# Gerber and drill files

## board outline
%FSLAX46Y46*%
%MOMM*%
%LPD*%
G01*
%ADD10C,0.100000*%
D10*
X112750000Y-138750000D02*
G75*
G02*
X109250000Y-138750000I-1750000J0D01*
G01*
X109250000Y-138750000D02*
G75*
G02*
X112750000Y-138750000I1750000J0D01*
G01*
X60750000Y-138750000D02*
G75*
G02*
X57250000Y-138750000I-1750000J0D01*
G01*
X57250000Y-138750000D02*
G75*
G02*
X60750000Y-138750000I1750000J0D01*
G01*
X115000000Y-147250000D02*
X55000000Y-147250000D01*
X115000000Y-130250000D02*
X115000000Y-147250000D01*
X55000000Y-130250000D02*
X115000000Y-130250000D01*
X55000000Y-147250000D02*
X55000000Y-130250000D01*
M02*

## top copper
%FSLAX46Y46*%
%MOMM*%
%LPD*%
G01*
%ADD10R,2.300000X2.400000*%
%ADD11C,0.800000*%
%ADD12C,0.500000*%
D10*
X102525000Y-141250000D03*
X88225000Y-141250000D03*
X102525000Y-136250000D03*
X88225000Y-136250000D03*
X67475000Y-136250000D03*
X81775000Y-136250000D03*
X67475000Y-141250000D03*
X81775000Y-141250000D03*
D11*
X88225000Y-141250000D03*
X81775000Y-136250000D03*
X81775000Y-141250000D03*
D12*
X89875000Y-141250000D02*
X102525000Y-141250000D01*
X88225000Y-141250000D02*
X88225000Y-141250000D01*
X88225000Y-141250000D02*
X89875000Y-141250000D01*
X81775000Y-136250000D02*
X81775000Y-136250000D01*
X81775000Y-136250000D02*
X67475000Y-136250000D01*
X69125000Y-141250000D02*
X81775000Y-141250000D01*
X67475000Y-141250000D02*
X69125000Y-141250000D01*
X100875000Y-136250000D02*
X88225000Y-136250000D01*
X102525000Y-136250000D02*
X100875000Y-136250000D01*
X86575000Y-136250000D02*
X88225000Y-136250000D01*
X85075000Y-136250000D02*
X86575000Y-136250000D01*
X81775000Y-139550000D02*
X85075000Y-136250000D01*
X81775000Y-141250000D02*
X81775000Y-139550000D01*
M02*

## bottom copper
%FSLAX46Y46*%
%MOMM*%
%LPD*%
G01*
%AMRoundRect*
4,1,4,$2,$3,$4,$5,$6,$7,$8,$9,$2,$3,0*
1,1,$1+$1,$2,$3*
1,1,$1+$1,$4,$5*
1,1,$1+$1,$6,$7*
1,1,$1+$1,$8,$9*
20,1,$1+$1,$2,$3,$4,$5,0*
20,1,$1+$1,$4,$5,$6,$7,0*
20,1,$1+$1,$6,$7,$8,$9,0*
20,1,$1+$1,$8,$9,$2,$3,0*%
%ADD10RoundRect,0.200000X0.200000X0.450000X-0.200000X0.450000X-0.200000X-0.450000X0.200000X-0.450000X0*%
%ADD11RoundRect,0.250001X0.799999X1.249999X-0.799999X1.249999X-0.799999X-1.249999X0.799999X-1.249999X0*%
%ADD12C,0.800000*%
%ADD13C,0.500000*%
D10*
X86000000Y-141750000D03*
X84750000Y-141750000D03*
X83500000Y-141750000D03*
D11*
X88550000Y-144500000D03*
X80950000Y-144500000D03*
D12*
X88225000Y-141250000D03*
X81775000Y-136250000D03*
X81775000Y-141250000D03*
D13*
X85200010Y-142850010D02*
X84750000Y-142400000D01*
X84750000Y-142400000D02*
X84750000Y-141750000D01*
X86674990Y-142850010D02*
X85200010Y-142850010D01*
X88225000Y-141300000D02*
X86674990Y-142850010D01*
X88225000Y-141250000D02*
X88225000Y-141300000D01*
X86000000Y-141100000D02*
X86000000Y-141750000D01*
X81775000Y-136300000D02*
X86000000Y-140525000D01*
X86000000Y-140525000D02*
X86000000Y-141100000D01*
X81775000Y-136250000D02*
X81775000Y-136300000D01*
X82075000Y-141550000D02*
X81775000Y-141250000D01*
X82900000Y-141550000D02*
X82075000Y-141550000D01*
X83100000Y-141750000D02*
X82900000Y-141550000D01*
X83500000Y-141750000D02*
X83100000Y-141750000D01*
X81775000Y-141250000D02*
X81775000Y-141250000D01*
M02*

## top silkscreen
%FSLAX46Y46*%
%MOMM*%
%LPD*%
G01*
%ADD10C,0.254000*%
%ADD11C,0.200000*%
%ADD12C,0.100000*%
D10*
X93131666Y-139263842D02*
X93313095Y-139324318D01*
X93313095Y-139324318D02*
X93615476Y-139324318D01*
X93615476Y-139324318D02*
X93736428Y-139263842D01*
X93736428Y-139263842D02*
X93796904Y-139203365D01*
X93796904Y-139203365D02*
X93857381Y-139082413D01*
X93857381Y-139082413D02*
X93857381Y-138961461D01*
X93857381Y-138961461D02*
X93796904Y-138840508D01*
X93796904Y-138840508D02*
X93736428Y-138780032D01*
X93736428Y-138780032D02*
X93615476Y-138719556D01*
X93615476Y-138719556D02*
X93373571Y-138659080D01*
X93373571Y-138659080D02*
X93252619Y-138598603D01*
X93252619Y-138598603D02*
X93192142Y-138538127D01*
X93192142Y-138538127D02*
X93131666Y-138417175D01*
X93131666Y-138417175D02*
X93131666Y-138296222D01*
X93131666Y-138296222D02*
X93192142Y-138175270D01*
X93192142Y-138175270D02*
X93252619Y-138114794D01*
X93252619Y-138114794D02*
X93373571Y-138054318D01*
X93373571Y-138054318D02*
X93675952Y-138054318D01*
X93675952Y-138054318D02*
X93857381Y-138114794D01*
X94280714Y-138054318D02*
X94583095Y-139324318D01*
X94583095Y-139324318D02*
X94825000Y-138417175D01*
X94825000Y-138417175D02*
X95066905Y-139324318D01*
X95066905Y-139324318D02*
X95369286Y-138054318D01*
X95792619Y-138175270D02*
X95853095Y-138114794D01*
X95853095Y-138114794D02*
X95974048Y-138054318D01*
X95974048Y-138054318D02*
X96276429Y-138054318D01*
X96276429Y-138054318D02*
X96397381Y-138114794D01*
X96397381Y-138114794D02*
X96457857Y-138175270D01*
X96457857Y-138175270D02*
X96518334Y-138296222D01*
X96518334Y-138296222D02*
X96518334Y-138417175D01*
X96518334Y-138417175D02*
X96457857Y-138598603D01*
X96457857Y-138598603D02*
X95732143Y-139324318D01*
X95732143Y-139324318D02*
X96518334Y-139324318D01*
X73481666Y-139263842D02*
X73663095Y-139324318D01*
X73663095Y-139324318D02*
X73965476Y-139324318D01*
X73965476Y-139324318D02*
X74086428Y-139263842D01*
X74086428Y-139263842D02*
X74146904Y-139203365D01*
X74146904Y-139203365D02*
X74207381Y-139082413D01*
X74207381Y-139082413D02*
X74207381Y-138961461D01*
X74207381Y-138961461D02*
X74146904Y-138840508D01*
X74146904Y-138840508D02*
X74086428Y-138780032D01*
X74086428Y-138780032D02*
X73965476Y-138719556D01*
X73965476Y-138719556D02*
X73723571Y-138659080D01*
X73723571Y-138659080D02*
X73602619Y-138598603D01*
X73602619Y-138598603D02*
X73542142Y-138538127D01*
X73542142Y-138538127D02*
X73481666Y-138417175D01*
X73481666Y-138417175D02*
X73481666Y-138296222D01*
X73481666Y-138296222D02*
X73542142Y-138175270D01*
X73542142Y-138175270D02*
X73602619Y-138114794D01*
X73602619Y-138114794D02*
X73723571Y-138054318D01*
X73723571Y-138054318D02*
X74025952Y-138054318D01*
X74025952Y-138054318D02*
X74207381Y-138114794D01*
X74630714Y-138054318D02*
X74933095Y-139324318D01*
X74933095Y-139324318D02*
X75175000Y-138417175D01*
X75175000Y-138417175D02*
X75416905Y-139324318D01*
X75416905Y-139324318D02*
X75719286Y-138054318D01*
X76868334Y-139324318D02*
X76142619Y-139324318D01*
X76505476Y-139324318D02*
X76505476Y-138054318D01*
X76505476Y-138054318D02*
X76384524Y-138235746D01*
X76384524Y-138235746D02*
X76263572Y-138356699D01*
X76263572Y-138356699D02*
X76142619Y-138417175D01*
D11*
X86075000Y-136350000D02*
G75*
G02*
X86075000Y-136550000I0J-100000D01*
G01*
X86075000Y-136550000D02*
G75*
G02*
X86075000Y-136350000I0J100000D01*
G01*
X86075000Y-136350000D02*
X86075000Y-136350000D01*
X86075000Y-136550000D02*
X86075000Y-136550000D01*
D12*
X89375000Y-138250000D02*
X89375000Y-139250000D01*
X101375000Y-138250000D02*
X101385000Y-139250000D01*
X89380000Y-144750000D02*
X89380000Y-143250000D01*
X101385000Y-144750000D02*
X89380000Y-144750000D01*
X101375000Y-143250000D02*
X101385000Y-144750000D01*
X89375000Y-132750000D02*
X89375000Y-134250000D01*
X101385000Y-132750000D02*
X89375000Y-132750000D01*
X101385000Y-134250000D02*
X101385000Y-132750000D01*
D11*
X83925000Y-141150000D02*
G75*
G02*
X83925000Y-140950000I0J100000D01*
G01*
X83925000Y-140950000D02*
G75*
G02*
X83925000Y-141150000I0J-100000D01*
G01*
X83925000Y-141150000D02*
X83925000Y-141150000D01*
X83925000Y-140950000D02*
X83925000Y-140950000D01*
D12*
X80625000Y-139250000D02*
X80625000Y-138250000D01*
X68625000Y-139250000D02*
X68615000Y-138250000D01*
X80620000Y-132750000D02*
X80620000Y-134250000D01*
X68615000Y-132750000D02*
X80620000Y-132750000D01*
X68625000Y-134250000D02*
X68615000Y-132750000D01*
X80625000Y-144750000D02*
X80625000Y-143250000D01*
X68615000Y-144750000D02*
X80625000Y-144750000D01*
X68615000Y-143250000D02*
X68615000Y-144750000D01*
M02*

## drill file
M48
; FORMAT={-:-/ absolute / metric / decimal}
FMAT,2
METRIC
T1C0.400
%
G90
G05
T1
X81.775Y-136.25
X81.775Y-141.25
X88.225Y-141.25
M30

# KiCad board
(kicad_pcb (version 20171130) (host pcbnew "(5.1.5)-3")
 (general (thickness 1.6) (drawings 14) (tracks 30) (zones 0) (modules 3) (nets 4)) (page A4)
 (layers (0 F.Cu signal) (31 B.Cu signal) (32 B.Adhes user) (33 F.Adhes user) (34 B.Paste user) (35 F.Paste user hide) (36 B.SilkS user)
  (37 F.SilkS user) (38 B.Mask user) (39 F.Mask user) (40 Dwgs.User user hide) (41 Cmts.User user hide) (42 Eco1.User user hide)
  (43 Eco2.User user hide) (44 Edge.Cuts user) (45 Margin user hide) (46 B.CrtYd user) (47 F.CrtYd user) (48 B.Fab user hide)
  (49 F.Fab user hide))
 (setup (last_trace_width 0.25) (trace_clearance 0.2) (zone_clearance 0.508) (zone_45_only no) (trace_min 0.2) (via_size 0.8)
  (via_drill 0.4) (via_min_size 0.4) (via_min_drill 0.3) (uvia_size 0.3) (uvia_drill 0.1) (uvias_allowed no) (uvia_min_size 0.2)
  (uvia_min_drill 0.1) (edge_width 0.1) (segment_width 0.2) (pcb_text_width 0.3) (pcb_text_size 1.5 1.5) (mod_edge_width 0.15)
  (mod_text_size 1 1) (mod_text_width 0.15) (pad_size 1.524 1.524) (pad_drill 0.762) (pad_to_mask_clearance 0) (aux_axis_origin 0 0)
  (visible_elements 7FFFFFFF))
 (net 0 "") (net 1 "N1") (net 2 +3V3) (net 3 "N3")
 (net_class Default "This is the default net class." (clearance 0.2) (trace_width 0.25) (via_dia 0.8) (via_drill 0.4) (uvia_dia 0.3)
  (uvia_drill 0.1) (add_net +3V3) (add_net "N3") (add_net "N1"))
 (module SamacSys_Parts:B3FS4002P (layer F.Cu) (at 94.25 138.75 180)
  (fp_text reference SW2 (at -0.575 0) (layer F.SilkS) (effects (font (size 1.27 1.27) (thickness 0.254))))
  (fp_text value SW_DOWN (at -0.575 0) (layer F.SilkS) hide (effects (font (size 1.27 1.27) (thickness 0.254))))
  (fp_arc (start 8.175 2.3) (end 8.175 2.4) (angle 180) (layer F.SilkS) (width 0.2))
  (fp_arc (start 8.175 2.3) (end 8.175 2.2) (angle 180) (layer F.SilkS) (width 0.2))
  (fp_line (start 8.175 2.4) (end 8.175 2.4) (layer F.SilkS) (width 0.2))
  (fp_line (start 8.175 2.2) (end 8.175 2.2) (layer F.SilkS) (width 0.2))
  (fp_line (start 4.875 0.5) (end 4.875 -0.5) (layer F.SilkS) (width 0.1))
  (fp_line (start -7.125 0.5) (end -7.135 -0.5) (layer F.SilkS) (width 0.1))
  (fp_line (start 4.87 -6) (end 4.87 -4.5) (layer F.SilkS) (width 0.1))
  (fp_line (start -7.135 -6) (end 4.87 -6) (layer F.SilkS) (width 0.1))
  (fp_line (start -7.125 -4.5) (end -7.135 -6) (layer F.SilkS) (width 0.1))
  (fp_line (start 4.875 6) (end 4.875 4.5) (layer F.SilkS) (width 0.1))
  (fp_line (start -7.135 6) (end 4.875 6) (layer F.SilkS) (width 0.1))
  (fp_line (start -7.135 4.5) (end -7.135 6) (layer F.SilkS) (width 0.1))
  (pad 2 smd rect (at -8.275 -2.5 180) (size 2.3 2.4) (layers F.Cu F.Paste F.Mask) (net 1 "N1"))
  (pad 2 smd rect (at 6.025 -2.5 180) (size 2.3 2.4) (layers F.Cu F.Paste F.Mask) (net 1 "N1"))
  (pad 1 smd rect (at -8.275 2.5 180) (size 2.3 2.4) (layers F.Cu F.Paste F.Mask) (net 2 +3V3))
  (pad 1 smd rect (at 6.025 2.5 180) (size 2.3 2.4) (layers F.Cu F.Paste F.Mask) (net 2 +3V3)))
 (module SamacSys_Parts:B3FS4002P (layer F.Cu) (at 75.75 138.75)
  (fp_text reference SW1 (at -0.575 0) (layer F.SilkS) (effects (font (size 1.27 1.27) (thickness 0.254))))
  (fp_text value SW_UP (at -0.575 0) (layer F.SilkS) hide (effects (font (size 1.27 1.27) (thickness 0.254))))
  (fp_arc (start 8.175 2.3) (end 8.175 2.4) (angle 180) (layer F.SilkS) (width 0.2))
  (fp_arc (start 8.175 2.3) (end 8.175 2.2) (angle 180) (layer F.SilkS) (width 0.2))
  (fp_line (start 8.175 2.4) (end 8.175 2.4) (layer F.SilkS) (width 0.2))
  (fp_line (start 8.175 2.2) (end 8.175 2.2) (layer F.SilkS) (width 0.2))
  (fp_line (start 4.875 0.5) (end 4.875 -0.5) (layer F.SilkS) (width 0.1))
  (fp_line (start -7.125 0.5) (end -7.135 -0.5) (layer F.SilkS) (width 0.1))
  (fp_line (start 4.87 -6) (end 4.87 -4.5) (layer F.SilkS) (width 0.1))
  (fp_line (start -7.135 -6) (end 4.87 -6) (layer F.SilkS) (width 0.1))
  (fp_line (start -7.125 -4.5) (end -7.135 -6) (layer F.SilkS) (width 0.1))
  (fp_line (start 4.875 6) (end 4.875 4.5) (layer F.SilkS) (width 0.1))
  (fp_line (start -7.135 6) (end 4.875 6) (layer F.SilkS) (width 0.1))
  (fp_line (start -7.135 4.5) (end -7.135 6) (layer F.SilkS) (width 0.1))
  (pad 2 smd rect (at -8.275 -2.5) (size 2.3 2.4) (layers F.Cu F.Paste F.Mask) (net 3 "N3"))
  (pad 2 smd rect (at 6.025 -2.5) (size 2.3 2.4) (layers F.Cu F.Paste F.Mask) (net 3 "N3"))
  (pad 1 smd rect (at -8.275 2.5) (size 2.3 2.4) (layers F.Cu F.Paste F.Mask) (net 2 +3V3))
  (pad 1 smd rect (at 6.025 2.5) (size 2.3 2.4) (layers F.Cu F.Paste F.Mask) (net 2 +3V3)))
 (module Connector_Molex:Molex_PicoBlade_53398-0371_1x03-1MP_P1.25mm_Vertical (layer B.Cu) (at 84.75 143 180)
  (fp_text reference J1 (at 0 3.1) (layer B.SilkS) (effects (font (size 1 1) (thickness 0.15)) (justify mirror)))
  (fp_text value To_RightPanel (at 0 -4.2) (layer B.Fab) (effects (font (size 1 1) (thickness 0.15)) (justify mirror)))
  (pad 1 smd roundrect (at -1.25 1.25 180) (size 0.8 1.3) (layers B.Cu B.Paste B.Mask) (roundrect_rratio 0.25) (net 3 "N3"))
  (pad 2 smd roundrect (at 0 1.25 180) (size 0.8 1.3) (layers B.Cu B.Paste B.Mask) (roundrect_rratio 0.25) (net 1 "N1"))
  (pad 3 smd roundrect (at 1.25 1.25 180) (size 0.8 1.3) (layers B.Cu B.Paste B.Mask) (roundrect_rratio 0.25) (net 2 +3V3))
  (pad MP smd roundrect (at -3.8 -1.5 180) (size 2.1 3) (layers B.Cu B.Paste B.Mask) (roundrect_rratio 0.119048))
  (pad MP smd roundrect (at 3.8 -1.5 180) (size 2.1 3) (layers B.Cu B.Paste B.Mask) (roundrect_rratio 0.119048)))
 (gr_circle (center 111 138.75) (end 111 140.5) (layer Edge.Cuts) (width 0.1))
 (gr_circle (center 59 138.75) (end 59 140.5) (layer Edge.Cuts) (width 0.1))
 (gr_line (start 115 147.25) (end 55 147.25) (layer Edge.Cuts) (width 0.1))
 (gr_line (start 115 130.25) (end 115 147.25) (layer Edge.Cuts) (width 0.1))
 (gr_line (start 55 130.25) (end 115 130.25) (layer Edge.Cuts) (width 0.1))
 (gr_line (start 55 147.25) (end 55 130.25) (layer Edge.Cuts) (width 0.1))
 (segment (start 89.875 141.25) (end 102.525 141.25) (width 0.5) (layer F.Cu) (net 1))
 (segment (start 88.225 141.25) (end 88.225 141.25) (width 0.5) (layer F.Cu) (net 1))
 (segment (start 88.225 141.25) (end 89.875 141.25) (width 0.5) (layer F.Cu) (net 1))
 (via (at 88.225 141.25) (size 0.8) (drill 0.4) (layers F.Cu B.Cu) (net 1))
 (segment (start 85.20001 142.85001) (end 84.75 142.4) (width 0.5) (layer B.Cu) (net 1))
 (segment (start 84.75 142.4) (end 84.75 141.75) (width 0.5) (layer B.Cu) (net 1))
 (segment (start 86.67499 142.85001) (end 85.20001 142.85001) (width 0.5) (layer B.Cu) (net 1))
 (segment (start 88.225 141.3) (end 86.67499 142.85001) (width 0.5) (layer B.Cu) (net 1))
 (segment (start 88.225 141.25) (end 88.225 141.3) (width 0.5) (layer B.Cu) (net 1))
 (segment (start 81.775 136.25) (end 81.775 136.25) (width 0.5) (layer F.Cu) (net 3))
 (segment (start 81.775 136.25) (end 67.475 136.25) (width 0.5) (layer F.Cu) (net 3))
 (via (at 81.775 136.25) (size 0.8) (drill 0.4) (layers F.Cu B.Cu) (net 3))
 (segment (start 86 141.1) (end 86 141.75) (width 0.5) (layer B.Cu) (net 3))
 (segment (start 81.775 136.3) (end 86 140.525) (width 0.5) (layer B.Cu) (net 3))
 (segment (start 86 140.525) (end 86 141.1) (width 0.5) (layer B.Cu) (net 3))
 (segment (start 81.775 136.25) (end 81.775 136.3) (width 0.5) (layer B.Cu) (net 3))
 (segment (start 82.075 141.55) (end 81.775 141.25) (width 0.5) (layer B.Cu) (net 2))
 (segment (start 69.125 141.25) (end 81.775 141.25) (width 0.5) (layer F.Cu) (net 2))
 (segment (start 67.475 141.25) (end 69.125 141.25) (width 0.5) (layer F.Cu) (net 2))
 (segment (start 100.875 136.25) (end 88.225 136.25) (width 0.5) (layer F.Cu) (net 2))
 (segment (start 102.525 136.25) (end 100.875 136.25) (width 0.5) (layer F.Cu) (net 2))
 (segment (start 86.575 136.25) (end 88.225 136.25) (width 0.5) (layer F.Cu) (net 2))
 (segment (start 85.075 136.25) (end 86.575 136.25) (width 0.5) (layer F.Cu) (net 2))
 (segment (start 81.775 139.55) (end 85.075 136.25) (width 0.5) (layer F.Cu) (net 2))
 (segment (start 81.775 141.25) (end 81.775 139.55) (width 0.5) (layer F.Cu) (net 2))
 (segment (start 82.9 141.55) (end 82.075 141.55) (width 0.5) (layer B.Cu) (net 2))
 (segment (start 83.1 141.75) (end 82.9 141.55) (width 0.5) (layer B.Cu) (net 2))
 (segment (start 83.5 141.75) (end 83.1 141.75) (width 0.5) (layer B.Cu) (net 2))
 (segment (start 81.775 141.25) (end 81.775 141.25) (width 0.5) (layer B.Cu) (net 2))
 (via (at 81.775 141.25) (size 0.8) (drill 0.4) (layers F.Cu B.Cu) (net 2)))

